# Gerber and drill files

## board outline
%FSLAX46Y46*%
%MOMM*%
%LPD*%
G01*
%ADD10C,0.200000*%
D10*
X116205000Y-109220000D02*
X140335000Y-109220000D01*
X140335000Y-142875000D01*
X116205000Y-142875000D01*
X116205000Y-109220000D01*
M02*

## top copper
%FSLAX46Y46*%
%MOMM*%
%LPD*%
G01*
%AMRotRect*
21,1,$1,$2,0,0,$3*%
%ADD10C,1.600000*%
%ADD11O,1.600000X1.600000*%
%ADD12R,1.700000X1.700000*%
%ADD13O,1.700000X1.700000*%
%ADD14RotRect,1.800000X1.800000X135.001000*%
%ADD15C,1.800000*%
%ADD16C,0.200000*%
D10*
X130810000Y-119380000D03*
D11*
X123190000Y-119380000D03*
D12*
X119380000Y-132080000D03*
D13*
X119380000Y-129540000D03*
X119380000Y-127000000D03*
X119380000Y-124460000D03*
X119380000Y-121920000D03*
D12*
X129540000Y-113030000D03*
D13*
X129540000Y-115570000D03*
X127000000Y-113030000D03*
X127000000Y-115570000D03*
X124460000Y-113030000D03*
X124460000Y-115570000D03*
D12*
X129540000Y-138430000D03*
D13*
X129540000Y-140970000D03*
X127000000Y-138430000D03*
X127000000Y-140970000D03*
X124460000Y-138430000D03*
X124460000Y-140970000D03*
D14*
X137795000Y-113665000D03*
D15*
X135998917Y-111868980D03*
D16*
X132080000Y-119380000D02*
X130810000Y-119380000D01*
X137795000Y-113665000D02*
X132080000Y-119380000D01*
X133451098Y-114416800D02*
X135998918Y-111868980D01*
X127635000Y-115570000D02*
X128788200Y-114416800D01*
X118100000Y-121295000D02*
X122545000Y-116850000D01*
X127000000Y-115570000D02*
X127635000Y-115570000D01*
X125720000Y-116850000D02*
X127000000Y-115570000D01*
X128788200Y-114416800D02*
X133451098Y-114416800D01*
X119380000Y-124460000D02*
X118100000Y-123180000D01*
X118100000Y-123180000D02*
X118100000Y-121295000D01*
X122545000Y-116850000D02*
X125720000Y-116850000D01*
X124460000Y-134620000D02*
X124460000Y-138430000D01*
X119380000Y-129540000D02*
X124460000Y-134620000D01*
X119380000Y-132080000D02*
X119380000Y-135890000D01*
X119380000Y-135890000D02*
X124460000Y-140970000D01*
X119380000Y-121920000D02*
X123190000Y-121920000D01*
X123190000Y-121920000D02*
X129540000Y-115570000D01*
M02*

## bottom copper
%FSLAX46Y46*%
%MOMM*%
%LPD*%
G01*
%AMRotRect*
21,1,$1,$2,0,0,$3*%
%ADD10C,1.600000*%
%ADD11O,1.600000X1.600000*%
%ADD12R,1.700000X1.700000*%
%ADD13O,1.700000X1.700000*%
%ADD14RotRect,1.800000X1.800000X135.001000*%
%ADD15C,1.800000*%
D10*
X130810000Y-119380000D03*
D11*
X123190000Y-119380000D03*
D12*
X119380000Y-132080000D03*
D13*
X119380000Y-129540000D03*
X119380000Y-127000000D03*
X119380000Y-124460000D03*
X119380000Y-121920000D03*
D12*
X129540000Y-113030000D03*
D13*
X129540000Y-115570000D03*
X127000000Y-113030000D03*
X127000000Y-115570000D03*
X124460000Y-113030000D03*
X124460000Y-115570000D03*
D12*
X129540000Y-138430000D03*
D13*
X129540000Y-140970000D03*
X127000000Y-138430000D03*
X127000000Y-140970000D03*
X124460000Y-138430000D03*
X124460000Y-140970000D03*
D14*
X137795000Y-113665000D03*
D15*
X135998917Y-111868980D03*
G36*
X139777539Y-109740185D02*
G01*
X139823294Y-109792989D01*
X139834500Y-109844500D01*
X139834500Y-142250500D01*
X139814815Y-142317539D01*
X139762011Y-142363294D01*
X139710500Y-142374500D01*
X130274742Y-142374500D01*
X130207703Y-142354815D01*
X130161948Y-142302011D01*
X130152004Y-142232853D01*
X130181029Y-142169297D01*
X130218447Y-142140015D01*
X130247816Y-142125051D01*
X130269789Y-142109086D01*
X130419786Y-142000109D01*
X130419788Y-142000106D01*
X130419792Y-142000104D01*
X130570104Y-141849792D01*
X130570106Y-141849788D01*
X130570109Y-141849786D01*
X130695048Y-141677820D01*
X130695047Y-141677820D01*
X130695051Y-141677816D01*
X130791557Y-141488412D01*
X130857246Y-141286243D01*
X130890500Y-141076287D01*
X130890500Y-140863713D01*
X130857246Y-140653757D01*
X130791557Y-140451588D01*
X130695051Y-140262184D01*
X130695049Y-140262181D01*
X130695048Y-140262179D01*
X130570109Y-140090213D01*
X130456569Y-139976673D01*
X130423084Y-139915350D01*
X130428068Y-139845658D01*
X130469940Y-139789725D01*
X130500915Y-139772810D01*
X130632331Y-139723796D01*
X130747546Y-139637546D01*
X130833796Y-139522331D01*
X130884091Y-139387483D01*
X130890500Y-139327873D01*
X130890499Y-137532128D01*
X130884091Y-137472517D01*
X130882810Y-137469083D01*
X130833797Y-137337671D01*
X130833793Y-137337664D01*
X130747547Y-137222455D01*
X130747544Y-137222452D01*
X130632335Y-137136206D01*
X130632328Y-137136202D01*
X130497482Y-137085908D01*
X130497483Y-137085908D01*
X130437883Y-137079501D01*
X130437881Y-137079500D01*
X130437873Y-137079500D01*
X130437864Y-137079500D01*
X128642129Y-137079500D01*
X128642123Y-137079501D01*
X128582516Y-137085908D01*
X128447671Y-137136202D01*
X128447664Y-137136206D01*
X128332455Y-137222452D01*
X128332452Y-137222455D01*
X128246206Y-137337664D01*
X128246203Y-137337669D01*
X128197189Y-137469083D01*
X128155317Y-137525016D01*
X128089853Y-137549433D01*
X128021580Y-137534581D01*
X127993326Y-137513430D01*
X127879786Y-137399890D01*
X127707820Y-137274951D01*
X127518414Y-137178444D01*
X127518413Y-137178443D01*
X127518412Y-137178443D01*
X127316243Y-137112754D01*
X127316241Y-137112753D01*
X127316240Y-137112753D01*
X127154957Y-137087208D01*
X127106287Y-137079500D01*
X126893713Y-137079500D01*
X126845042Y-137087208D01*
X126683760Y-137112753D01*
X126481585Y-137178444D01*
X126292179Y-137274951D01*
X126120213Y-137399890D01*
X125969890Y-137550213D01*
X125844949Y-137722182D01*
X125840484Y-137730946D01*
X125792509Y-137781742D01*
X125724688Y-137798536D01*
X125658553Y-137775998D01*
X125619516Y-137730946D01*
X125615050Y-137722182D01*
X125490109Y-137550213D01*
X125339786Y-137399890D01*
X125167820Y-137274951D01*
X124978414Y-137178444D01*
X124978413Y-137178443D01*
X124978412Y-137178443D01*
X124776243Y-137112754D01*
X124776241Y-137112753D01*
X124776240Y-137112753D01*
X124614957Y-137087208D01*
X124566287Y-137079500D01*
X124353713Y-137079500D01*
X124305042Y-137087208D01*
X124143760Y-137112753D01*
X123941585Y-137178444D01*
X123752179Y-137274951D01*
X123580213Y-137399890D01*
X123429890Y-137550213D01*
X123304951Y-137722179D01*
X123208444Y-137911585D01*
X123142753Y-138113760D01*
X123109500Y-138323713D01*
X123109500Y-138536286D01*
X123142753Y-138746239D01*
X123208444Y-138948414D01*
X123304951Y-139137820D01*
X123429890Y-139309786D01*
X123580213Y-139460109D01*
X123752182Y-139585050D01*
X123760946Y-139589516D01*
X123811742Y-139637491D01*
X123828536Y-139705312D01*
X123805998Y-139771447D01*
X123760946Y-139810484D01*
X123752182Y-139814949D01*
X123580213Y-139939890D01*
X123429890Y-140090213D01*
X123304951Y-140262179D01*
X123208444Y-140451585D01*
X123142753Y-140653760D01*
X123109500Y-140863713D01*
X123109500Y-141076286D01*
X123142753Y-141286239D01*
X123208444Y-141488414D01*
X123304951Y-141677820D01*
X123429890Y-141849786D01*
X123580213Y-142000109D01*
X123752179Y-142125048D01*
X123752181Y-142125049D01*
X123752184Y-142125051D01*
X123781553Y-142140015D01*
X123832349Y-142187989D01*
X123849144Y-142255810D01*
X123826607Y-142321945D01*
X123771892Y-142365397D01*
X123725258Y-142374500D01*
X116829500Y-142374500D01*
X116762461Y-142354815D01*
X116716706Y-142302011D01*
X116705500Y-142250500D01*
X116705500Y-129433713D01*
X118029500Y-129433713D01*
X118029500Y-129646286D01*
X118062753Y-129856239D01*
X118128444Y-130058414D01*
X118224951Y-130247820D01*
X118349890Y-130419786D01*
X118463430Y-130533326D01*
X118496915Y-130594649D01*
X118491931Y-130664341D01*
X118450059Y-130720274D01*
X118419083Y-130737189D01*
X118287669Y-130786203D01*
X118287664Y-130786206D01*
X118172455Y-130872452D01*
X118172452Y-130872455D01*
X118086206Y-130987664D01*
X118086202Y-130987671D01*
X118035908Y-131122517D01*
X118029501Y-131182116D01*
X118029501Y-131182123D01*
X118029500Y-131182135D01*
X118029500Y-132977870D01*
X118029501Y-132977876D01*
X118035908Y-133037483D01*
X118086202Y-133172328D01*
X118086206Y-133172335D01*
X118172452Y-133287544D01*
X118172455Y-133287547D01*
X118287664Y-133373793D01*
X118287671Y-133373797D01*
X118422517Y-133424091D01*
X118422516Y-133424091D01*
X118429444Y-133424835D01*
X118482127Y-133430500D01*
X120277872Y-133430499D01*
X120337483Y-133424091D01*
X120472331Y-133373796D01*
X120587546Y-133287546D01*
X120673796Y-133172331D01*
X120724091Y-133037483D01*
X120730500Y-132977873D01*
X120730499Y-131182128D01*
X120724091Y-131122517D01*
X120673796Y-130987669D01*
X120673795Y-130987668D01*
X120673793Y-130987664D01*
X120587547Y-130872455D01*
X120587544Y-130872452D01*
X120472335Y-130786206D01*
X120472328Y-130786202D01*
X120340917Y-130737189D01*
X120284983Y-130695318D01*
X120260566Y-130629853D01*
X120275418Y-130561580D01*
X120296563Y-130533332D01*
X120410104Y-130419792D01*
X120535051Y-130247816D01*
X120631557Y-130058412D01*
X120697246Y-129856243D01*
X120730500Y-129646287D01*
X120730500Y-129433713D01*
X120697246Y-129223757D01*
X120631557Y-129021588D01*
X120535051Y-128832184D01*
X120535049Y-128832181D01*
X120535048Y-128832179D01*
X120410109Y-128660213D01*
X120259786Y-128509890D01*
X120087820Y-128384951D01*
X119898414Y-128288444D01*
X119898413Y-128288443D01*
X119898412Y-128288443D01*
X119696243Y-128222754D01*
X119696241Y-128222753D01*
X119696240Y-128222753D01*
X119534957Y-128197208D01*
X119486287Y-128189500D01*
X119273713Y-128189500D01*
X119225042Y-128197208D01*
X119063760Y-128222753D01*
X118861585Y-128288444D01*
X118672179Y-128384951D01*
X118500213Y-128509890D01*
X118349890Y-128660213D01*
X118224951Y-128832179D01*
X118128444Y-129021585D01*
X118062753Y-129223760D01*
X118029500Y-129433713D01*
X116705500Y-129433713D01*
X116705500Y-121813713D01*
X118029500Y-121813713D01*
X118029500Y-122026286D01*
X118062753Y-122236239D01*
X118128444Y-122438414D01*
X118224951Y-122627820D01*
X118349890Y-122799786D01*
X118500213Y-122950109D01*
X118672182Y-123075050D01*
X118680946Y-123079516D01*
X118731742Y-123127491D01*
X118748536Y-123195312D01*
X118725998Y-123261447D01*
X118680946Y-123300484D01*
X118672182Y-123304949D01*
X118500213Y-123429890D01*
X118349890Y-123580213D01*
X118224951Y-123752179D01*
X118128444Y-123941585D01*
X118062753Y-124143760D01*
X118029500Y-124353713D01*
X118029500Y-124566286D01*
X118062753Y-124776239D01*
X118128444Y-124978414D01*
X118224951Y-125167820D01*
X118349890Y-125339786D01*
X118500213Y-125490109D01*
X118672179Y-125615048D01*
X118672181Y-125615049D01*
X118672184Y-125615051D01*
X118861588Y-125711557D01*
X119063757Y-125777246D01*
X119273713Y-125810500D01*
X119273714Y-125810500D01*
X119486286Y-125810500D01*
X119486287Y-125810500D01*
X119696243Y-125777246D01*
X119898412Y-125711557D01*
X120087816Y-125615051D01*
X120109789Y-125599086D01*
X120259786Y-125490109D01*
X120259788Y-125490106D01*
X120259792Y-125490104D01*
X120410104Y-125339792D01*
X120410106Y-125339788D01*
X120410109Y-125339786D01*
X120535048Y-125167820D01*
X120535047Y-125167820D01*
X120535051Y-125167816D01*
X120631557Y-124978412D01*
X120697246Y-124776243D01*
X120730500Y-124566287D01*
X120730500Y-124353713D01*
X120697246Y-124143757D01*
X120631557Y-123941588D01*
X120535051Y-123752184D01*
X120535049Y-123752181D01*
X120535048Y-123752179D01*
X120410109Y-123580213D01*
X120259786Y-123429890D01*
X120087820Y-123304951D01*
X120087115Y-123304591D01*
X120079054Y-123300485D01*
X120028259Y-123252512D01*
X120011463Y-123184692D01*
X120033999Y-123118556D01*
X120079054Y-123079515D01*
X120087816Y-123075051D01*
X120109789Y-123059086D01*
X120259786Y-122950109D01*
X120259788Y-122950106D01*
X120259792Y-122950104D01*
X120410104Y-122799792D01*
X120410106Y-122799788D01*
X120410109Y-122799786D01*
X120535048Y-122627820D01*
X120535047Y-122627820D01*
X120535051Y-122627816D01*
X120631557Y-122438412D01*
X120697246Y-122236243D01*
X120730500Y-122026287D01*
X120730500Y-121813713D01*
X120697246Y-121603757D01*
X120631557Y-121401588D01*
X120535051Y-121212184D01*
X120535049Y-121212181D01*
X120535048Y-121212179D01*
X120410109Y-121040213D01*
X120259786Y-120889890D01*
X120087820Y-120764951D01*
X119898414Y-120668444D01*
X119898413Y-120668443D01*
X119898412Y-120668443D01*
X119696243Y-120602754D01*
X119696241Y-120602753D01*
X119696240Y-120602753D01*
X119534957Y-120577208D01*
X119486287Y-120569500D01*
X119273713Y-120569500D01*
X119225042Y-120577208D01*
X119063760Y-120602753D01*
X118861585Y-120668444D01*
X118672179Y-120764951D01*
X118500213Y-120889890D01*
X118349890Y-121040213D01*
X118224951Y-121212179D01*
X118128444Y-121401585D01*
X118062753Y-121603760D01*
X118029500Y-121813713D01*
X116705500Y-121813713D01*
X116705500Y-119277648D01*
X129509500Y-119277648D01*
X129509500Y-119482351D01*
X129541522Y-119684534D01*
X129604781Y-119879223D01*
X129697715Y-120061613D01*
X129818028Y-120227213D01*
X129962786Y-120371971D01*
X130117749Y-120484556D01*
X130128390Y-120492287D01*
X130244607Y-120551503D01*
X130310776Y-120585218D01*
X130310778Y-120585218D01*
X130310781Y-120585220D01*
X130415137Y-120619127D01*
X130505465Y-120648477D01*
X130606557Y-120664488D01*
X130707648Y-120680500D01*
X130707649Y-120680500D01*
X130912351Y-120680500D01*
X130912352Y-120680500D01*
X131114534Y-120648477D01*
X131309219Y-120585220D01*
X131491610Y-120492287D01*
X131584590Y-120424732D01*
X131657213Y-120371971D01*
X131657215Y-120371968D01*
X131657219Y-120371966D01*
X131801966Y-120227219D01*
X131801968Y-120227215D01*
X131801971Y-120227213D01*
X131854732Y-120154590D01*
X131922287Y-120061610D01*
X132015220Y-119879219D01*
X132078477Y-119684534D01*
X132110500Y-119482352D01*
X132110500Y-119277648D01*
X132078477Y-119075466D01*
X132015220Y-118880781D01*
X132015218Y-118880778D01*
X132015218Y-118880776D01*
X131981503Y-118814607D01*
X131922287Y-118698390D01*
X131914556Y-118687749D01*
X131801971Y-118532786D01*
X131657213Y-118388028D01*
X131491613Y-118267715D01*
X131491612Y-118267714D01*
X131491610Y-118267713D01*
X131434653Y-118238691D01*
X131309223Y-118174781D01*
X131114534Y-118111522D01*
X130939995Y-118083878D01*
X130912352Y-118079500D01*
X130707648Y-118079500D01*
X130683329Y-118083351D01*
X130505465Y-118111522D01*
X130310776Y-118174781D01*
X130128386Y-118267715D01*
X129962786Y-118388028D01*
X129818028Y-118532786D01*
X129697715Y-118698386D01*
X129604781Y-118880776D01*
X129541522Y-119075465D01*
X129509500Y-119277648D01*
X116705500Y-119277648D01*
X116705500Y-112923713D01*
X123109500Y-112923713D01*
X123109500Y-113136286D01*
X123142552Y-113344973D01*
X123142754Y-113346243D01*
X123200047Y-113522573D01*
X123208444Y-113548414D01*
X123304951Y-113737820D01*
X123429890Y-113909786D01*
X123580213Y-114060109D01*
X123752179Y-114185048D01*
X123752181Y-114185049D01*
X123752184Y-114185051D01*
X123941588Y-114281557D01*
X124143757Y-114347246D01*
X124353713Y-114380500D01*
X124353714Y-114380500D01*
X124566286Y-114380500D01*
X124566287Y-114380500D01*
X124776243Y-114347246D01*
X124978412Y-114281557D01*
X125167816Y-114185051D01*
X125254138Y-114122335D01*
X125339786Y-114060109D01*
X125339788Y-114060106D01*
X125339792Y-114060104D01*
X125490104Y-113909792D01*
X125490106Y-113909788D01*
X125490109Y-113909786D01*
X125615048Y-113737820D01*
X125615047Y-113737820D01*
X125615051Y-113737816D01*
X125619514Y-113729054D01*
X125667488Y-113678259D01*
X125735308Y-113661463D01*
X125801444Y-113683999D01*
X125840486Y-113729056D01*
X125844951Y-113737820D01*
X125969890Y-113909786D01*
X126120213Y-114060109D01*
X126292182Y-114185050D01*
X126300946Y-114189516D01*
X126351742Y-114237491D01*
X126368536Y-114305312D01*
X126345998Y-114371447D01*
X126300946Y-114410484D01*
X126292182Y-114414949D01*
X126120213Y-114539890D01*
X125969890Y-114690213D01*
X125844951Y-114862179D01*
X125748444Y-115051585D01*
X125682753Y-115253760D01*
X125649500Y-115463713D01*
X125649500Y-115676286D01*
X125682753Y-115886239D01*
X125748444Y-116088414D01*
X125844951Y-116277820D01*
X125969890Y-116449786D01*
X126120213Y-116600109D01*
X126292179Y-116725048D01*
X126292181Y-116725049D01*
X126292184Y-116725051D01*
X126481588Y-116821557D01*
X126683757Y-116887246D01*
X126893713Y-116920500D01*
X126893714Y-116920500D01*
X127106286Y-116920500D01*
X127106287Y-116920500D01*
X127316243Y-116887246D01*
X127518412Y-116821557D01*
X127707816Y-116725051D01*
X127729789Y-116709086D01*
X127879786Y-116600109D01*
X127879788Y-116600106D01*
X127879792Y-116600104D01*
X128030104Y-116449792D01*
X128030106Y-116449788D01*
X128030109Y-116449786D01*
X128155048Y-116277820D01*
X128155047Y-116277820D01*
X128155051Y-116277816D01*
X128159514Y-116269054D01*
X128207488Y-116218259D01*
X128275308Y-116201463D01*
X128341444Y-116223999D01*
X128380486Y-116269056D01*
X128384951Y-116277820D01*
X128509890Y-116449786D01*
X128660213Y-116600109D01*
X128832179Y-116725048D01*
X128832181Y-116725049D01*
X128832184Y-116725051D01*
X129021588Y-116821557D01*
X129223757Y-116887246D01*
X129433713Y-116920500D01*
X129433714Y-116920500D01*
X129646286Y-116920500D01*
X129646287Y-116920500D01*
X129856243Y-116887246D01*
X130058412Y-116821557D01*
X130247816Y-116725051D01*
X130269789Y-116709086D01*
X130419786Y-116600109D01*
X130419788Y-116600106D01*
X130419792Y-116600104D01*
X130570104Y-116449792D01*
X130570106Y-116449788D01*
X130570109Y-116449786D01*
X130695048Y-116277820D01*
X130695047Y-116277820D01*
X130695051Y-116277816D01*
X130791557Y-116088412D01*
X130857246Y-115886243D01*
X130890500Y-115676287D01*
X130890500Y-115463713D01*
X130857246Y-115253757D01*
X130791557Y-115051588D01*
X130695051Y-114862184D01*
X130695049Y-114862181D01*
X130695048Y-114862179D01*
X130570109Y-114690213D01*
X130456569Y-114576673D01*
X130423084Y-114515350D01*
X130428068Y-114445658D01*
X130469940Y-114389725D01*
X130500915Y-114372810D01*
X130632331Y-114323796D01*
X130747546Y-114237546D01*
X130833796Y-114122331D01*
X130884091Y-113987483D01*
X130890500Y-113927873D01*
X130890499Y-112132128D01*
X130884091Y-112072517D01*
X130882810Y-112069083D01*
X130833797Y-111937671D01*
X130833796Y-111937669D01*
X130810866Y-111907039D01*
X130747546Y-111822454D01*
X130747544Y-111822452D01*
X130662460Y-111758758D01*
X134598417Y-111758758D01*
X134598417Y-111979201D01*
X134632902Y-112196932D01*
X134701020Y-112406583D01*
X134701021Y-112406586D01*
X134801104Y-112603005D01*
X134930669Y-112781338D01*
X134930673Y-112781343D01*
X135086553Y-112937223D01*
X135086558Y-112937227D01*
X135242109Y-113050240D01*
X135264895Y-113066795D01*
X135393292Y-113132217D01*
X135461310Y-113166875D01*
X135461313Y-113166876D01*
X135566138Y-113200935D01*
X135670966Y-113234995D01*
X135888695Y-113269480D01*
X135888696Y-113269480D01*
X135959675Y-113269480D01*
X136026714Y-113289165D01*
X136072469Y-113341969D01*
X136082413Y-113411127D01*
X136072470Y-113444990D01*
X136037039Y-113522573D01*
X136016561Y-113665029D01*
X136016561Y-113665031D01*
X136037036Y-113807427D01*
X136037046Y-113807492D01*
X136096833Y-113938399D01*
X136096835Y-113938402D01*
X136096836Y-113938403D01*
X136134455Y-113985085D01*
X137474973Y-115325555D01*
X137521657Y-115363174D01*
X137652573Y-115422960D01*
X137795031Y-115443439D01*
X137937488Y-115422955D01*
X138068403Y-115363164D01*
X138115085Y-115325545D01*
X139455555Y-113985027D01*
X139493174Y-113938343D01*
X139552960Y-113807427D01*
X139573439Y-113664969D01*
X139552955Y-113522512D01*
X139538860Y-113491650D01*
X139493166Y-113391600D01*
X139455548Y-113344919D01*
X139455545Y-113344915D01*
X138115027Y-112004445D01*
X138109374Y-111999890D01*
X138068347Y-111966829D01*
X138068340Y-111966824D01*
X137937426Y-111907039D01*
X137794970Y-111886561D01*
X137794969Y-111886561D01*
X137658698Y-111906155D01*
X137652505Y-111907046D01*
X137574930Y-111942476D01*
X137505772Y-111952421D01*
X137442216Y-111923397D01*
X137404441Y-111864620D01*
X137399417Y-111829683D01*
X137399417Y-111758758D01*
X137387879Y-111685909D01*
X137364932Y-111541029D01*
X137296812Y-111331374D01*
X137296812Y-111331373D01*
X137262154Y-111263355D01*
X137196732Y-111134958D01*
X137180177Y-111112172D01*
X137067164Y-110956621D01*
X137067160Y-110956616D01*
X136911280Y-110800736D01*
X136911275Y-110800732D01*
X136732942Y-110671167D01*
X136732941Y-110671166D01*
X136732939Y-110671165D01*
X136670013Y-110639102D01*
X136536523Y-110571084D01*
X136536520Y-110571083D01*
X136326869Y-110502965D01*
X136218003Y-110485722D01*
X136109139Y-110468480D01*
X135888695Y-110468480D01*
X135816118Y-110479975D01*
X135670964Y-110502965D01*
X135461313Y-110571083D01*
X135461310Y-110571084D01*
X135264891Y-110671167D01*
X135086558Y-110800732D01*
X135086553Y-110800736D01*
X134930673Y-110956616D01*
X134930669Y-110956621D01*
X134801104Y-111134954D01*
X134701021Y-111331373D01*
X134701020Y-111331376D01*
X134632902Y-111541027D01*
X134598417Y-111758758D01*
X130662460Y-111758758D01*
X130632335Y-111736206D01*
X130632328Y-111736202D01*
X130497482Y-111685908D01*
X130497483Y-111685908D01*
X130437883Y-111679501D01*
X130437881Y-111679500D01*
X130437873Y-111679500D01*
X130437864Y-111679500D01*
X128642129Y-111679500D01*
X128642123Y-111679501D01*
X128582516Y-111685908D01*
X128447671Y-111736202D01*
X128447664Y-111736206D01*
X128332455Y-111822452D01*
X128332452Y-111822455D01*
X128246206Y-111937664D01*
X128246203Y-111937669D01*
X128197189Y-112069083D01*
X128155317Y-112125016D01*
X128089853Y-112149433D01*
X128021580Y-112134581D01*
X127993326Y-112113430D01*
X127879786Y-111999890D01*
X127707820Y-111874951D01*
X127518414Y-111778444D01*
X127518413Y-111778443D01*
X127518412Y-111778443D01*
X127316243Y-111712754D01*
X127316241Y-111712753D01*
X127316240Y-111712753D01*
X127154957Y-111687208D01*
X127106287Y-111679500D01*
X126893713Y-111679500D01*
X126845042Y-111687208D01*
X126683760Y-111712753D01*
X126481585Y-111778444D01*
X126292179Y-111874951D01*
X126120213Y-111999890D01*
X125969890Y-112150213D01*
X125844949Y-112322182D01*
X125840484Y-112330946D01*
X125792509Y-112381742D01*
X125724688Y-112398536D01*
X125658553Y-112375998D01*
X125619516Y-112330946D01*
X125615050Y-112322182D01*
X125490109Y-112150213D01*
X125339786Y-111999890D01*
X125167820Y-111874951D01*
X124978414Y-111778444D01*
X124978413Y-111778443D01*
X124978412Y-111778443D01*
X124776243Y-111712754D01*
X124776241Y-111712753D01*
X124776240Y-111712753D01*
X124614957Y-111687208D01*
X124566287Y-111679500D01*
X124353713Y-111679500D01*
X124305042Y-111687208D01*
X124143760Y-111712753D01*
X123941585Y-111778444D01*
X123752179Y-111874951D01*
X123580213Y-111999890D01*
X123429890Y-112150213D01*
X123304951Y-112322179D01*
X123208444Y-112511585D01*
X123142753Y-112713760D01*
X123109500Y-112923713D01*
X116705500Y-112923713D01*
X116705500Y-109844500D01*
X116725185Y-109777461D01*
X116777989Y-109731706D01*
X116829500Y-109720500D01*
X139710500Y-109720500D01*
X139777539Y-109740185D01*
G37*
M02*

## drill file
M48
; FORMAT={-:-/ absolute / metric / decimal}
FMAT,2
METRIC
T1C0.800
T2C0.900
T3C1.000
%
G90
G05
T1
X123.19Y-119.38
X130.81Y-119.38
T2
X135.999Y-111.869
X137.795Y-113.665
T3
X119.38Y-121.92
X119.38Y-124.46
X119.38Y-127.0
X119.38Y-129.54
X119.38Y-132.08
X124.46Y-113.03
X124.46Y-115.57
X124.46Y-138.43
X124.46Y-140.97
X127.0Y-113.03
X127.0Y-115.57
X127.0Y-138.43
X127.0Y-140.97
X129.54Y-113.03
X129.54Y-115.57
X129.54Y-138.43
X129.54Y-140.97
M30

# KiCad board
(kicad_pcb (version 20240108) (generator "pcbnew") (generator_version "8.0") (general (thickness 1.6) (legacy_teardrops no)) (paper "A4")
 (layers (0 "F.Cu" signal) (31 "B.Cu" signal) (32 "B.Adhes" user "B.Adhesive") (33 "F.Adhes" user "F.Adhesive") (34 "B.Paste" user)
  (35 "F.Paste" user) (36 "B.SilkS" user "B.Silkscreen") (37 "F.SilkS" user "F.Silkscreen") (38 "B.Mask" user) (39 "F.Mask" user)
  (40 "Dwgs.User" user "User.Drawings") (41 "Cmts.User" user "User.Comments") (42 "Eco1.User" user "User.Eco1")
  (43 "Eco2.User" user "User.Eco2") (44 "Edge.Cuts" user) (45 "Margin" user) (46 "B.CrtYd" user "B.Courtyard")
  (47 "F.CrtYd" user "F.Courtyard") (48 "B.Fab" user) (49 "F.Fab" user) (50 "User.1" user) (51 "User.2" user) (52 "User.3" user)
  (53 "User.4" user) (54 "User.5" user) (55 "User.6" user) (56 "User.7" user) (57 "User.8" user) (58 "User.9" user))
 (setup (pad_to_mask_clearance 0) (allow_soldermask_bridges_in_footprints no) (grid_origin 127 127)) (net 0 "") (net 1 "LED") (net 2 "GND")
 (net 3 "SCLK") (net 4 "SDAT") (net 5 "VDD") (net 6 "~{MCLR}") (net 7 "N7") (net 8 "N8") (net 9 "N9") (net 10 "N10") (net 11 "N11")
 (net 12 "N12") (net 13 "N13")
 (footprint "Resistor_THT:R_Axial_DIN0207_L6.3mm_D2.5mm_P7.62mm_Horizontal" (layer "F.Cu") (at 130.81 119.38 180)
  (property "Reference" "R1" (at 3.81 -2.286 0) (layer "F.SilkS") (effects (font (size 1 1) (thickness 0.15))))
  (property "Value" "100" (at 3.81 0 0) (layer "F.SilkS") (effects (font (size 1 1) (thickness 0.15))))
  (pad "1" thru_hole circle (at 0 0 180) (size 1.6 1.6) (drill 0.8) (layers "*.Cu" "*.Mask") (remove_unused_layers no) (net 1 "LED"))
  (pad "2" thru_hole oval (at 7.62 0 180) (size 1.6 1.6) (drill 0.8) (layers "*.Cu" "*.Mask") (remove_unused_layers no) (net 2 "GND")))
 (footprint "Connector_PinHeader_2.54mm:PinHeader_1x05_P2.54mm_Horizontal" (layer "F.Cu") (at 119.38 132.08 180)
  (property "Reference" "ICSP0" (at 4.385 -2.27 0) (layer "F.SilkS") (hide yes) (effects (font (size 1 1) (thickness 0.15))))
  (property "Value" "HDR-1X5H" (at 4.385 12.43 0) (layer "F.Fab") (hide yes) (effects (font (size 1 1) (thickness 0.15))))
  (pad "1" thru_hole rect (at 0 0 180) (size 1.7 1.7) (drill 1) (layers "*.Cu" "*.Mask") (remove_unused_layers no) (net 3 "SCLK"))
  (pad "2" thru_hole oval (at 0 2.54 180) (size 1.7 1.7) (drill 1) (layers "*.Cu" "*.Mask") (remove_unused_layers no) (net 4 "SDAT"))
  (pad "3" thru_hole oval (at 0 5.08 180) (size 1.7 1.7) (drill 1) (layers "*.Cu" "*.Mask") (remove_unused_layers no) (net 2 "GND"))
  (pad "4" thru_hole oval (at 0 7.62 180) (size 1.7 1.7) (drill 1) (layers "*.Cu" "*.Mask") (remove_unused_layers no) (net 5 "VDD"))
  (pad "5" thru_hole oval (at 0 10.16 180) (size 1.7 1.7) (drill 1) (layers "*.Cu" "*.Mask") (remove_unused_layers no) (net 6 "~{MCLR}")))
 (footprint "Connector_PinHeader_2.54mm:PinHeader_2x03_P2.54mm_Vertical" (layer "F.Cu") (at 129.54 113.03 -90)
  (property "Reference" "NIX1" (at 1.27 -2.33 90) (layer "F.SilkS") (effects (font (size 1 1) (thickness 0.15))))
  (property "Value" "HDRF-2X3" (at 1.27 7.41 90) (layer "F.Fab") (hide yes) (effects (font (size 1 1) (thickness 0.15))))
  (pad "1" thru_hole rect (at 0 0 270) (size 1.7 1.7) (drill 1) (layers "*.Cu" "*.Mask") (remove_unused_layers no) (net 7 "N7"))
  (pad "2" thru_hole oval (at 2.54 0 270) (size 1.7 1.7) (drill 1) (layers "*.Cu" "*.Mask") (remove_unused_layers no) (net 6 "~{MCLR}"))
  (pad "3" thru_hole oval (at 0 2.54 270) (size 1.7 1.7) (drill 1) (layers "*.Cu" "*.Mask") (remove_unused_layers no) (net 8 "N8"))
  (pad "4" thru_hole oval (at 2.54 2.54 270) (size 1.7 1.7) (drill 1) (layers "*.Cu" "*.Mask") (remove_unused_layers no) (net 5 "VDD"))
  (pad "5" thru_hole oval (at 0 5.08 270) (size 1.7 1.7) (drill 1) (layers "*.Cu" "*.Mask") (remove_unused_layers no) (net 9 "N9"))
  (pad "6" thru_hole oval (at 2.54 5.08 270) (size 1.7 1.7) (drill 1) (layers "*.Cu" "*.Mask") (remove_unused_layers no) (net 2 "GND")))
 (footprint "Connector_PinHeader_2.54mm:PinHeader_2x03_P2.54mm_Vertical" (layer "F.Cu") (at 129.54 138.43 -90)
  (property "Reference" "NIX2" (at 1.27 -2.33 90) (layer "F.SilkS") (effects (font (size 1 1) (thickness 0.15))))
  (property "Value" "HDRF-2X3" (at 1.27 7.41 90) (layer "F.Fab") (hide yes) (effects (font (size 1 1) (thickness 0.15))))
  (pad "1" thru_hole rect (at 0 0 270) (size 1.7 1.7) (drill 1) (layers "*.Cu" "*.Mask") (remove_unused_layers no) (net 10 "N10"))
  (pad "2" thru_hole oval (at 2.54 0 270) (size 1.7 1.7) (drill 1) (layers "*.Cu" "*.Mask") (remove_unused_layers no) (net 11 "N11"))
  (pad "3" thru_hole oval (at 0 2.54 270) (size 1.7 1.7) (drill 1) (layers "*.Cu" "*.Mask") (remove_unused_layers no) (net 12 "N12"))
  (pad "4" thru_hole oval (at 2.54 2.54 270) (size 1.7 1.7) (drill 1) (layers "*.Cu" "*.Mask") (remove_unused_layers no) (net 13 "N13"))
  (pad "5" thru_hole oval (at 0 5.08 270) (size 1.7 1.7) (drill 1) (layers "*.Cu" "*.Mask") (remove_unused_layers no) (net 4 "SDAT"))
  (pad "6" thru_hole oval (at 2.54 5.08 270) (size 1.7 1.7) (drill 1) (layers "*.Cu" "*.Mask") (remove_unused_layers no) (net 3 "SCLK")))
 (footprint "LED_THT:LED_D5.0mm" (layer "F.Cu") (at 137.795 113.665 135.001)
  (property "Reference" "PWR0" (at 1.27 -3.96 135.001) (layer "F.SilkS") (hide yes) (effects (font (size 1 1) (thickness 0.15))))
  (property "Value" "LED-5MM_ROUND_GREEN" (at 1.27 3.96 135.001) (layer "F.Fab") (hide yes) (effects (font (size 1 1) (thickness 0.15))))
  (pad "1" thru_hole rect (at 0 0 135.001) (size 1.8 1.8) (drill 0.9) (layers "*.Cu" "*.Mask") (remove_unused_layers no) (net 1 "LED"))
  (pad "2" thru_hole circle (at 2.54 0 135.001) (size 1.8 1.8) (drill 0.9) (layers "*.Cu" "*.Mask") (remove_unused_layers no) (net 5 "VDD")))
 (gr_rect (start 116.205 109.22) (end 140.335 142.875) (stroke (width 0.2) (type default)) (fill none) (layer "Edge.Cuts"))
 (segment (start 132.08 119.38) (end 130.81 119.38) (width 0.2) (layer "F.Cu") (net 1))
 (segment (start 137.795 113.665) (end 132.08 119.38) (width 0.2) (layer "F.Cu") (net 1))
 (segment (start 133.451098 114.4168) (end 135.998918 111.86898) (width 0.2) (layer "F.Cu") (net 5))
 (segment (start 127.635 115.57) (end 128.7882 114.4168) (width 0.2) (layer "F.Cu") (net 5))
 (segment (start 118.1 121.295) (end 122.545 116.85) (width 0.2) (layer "F.Cu") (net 5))
 (segment (start 127 115.57) (end 127.635 115.57) (width 0.2) (layer "F.Cu") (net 5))
 (segment (start 125.72 116.85) (end 127 115.57) (width 0.2) (layer "F.Cu") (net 5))
 (segment (start 128.7882 114.4168) (end 133.451098 114.4168) (width 0.2) (layer "F.Cu") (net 5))
 (segment (start 119.38 124.46) (end 118.1 123.18) (width 0.2) (layer "F.Cu") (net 5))
 (segment (start 118.1 123.18) (end 118.1 121.295) (width 0.2) (layer "F.Cu") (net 5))
 (segment (start 122.545 116.85) (end 125.72 116.85) (width 0.2) (layer "F.Cu") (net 5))
 (segment (start 124.46 134.62) (end 124.46 138.43) (width 0.2) (layer "F.Cu") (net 4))
 (segment (start 119.38 129.54) (end 124.46 134.62) (width 0.2) (layer "F.Cu") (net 4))
 (segment (start 119.38 132.08) (end 119.38 135.89) (width 0.2) (layer "F.Cu") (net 3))
 (segment (start 119.38 135.89) (end 124.46 140.97) (width 0.2) (layer "F.Cu") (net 3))
 (segment (start 119.38 121.92) (end 123.19 121.92) (width 0.2) (layer "F.Cu") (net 6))
 (segment (start 123.19 121.92) (end 129.54 115.57) (width 0.2) (layer "F.Cu") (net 6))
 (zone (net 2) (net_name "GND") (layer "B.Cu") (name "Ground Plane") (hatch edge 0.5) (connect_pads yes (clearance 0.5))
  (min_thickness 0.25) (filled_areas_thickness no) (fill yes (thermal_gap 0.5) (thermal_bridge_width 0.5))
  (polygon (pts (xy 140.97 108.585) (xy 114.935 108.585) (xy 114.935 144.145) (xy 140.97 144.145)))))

